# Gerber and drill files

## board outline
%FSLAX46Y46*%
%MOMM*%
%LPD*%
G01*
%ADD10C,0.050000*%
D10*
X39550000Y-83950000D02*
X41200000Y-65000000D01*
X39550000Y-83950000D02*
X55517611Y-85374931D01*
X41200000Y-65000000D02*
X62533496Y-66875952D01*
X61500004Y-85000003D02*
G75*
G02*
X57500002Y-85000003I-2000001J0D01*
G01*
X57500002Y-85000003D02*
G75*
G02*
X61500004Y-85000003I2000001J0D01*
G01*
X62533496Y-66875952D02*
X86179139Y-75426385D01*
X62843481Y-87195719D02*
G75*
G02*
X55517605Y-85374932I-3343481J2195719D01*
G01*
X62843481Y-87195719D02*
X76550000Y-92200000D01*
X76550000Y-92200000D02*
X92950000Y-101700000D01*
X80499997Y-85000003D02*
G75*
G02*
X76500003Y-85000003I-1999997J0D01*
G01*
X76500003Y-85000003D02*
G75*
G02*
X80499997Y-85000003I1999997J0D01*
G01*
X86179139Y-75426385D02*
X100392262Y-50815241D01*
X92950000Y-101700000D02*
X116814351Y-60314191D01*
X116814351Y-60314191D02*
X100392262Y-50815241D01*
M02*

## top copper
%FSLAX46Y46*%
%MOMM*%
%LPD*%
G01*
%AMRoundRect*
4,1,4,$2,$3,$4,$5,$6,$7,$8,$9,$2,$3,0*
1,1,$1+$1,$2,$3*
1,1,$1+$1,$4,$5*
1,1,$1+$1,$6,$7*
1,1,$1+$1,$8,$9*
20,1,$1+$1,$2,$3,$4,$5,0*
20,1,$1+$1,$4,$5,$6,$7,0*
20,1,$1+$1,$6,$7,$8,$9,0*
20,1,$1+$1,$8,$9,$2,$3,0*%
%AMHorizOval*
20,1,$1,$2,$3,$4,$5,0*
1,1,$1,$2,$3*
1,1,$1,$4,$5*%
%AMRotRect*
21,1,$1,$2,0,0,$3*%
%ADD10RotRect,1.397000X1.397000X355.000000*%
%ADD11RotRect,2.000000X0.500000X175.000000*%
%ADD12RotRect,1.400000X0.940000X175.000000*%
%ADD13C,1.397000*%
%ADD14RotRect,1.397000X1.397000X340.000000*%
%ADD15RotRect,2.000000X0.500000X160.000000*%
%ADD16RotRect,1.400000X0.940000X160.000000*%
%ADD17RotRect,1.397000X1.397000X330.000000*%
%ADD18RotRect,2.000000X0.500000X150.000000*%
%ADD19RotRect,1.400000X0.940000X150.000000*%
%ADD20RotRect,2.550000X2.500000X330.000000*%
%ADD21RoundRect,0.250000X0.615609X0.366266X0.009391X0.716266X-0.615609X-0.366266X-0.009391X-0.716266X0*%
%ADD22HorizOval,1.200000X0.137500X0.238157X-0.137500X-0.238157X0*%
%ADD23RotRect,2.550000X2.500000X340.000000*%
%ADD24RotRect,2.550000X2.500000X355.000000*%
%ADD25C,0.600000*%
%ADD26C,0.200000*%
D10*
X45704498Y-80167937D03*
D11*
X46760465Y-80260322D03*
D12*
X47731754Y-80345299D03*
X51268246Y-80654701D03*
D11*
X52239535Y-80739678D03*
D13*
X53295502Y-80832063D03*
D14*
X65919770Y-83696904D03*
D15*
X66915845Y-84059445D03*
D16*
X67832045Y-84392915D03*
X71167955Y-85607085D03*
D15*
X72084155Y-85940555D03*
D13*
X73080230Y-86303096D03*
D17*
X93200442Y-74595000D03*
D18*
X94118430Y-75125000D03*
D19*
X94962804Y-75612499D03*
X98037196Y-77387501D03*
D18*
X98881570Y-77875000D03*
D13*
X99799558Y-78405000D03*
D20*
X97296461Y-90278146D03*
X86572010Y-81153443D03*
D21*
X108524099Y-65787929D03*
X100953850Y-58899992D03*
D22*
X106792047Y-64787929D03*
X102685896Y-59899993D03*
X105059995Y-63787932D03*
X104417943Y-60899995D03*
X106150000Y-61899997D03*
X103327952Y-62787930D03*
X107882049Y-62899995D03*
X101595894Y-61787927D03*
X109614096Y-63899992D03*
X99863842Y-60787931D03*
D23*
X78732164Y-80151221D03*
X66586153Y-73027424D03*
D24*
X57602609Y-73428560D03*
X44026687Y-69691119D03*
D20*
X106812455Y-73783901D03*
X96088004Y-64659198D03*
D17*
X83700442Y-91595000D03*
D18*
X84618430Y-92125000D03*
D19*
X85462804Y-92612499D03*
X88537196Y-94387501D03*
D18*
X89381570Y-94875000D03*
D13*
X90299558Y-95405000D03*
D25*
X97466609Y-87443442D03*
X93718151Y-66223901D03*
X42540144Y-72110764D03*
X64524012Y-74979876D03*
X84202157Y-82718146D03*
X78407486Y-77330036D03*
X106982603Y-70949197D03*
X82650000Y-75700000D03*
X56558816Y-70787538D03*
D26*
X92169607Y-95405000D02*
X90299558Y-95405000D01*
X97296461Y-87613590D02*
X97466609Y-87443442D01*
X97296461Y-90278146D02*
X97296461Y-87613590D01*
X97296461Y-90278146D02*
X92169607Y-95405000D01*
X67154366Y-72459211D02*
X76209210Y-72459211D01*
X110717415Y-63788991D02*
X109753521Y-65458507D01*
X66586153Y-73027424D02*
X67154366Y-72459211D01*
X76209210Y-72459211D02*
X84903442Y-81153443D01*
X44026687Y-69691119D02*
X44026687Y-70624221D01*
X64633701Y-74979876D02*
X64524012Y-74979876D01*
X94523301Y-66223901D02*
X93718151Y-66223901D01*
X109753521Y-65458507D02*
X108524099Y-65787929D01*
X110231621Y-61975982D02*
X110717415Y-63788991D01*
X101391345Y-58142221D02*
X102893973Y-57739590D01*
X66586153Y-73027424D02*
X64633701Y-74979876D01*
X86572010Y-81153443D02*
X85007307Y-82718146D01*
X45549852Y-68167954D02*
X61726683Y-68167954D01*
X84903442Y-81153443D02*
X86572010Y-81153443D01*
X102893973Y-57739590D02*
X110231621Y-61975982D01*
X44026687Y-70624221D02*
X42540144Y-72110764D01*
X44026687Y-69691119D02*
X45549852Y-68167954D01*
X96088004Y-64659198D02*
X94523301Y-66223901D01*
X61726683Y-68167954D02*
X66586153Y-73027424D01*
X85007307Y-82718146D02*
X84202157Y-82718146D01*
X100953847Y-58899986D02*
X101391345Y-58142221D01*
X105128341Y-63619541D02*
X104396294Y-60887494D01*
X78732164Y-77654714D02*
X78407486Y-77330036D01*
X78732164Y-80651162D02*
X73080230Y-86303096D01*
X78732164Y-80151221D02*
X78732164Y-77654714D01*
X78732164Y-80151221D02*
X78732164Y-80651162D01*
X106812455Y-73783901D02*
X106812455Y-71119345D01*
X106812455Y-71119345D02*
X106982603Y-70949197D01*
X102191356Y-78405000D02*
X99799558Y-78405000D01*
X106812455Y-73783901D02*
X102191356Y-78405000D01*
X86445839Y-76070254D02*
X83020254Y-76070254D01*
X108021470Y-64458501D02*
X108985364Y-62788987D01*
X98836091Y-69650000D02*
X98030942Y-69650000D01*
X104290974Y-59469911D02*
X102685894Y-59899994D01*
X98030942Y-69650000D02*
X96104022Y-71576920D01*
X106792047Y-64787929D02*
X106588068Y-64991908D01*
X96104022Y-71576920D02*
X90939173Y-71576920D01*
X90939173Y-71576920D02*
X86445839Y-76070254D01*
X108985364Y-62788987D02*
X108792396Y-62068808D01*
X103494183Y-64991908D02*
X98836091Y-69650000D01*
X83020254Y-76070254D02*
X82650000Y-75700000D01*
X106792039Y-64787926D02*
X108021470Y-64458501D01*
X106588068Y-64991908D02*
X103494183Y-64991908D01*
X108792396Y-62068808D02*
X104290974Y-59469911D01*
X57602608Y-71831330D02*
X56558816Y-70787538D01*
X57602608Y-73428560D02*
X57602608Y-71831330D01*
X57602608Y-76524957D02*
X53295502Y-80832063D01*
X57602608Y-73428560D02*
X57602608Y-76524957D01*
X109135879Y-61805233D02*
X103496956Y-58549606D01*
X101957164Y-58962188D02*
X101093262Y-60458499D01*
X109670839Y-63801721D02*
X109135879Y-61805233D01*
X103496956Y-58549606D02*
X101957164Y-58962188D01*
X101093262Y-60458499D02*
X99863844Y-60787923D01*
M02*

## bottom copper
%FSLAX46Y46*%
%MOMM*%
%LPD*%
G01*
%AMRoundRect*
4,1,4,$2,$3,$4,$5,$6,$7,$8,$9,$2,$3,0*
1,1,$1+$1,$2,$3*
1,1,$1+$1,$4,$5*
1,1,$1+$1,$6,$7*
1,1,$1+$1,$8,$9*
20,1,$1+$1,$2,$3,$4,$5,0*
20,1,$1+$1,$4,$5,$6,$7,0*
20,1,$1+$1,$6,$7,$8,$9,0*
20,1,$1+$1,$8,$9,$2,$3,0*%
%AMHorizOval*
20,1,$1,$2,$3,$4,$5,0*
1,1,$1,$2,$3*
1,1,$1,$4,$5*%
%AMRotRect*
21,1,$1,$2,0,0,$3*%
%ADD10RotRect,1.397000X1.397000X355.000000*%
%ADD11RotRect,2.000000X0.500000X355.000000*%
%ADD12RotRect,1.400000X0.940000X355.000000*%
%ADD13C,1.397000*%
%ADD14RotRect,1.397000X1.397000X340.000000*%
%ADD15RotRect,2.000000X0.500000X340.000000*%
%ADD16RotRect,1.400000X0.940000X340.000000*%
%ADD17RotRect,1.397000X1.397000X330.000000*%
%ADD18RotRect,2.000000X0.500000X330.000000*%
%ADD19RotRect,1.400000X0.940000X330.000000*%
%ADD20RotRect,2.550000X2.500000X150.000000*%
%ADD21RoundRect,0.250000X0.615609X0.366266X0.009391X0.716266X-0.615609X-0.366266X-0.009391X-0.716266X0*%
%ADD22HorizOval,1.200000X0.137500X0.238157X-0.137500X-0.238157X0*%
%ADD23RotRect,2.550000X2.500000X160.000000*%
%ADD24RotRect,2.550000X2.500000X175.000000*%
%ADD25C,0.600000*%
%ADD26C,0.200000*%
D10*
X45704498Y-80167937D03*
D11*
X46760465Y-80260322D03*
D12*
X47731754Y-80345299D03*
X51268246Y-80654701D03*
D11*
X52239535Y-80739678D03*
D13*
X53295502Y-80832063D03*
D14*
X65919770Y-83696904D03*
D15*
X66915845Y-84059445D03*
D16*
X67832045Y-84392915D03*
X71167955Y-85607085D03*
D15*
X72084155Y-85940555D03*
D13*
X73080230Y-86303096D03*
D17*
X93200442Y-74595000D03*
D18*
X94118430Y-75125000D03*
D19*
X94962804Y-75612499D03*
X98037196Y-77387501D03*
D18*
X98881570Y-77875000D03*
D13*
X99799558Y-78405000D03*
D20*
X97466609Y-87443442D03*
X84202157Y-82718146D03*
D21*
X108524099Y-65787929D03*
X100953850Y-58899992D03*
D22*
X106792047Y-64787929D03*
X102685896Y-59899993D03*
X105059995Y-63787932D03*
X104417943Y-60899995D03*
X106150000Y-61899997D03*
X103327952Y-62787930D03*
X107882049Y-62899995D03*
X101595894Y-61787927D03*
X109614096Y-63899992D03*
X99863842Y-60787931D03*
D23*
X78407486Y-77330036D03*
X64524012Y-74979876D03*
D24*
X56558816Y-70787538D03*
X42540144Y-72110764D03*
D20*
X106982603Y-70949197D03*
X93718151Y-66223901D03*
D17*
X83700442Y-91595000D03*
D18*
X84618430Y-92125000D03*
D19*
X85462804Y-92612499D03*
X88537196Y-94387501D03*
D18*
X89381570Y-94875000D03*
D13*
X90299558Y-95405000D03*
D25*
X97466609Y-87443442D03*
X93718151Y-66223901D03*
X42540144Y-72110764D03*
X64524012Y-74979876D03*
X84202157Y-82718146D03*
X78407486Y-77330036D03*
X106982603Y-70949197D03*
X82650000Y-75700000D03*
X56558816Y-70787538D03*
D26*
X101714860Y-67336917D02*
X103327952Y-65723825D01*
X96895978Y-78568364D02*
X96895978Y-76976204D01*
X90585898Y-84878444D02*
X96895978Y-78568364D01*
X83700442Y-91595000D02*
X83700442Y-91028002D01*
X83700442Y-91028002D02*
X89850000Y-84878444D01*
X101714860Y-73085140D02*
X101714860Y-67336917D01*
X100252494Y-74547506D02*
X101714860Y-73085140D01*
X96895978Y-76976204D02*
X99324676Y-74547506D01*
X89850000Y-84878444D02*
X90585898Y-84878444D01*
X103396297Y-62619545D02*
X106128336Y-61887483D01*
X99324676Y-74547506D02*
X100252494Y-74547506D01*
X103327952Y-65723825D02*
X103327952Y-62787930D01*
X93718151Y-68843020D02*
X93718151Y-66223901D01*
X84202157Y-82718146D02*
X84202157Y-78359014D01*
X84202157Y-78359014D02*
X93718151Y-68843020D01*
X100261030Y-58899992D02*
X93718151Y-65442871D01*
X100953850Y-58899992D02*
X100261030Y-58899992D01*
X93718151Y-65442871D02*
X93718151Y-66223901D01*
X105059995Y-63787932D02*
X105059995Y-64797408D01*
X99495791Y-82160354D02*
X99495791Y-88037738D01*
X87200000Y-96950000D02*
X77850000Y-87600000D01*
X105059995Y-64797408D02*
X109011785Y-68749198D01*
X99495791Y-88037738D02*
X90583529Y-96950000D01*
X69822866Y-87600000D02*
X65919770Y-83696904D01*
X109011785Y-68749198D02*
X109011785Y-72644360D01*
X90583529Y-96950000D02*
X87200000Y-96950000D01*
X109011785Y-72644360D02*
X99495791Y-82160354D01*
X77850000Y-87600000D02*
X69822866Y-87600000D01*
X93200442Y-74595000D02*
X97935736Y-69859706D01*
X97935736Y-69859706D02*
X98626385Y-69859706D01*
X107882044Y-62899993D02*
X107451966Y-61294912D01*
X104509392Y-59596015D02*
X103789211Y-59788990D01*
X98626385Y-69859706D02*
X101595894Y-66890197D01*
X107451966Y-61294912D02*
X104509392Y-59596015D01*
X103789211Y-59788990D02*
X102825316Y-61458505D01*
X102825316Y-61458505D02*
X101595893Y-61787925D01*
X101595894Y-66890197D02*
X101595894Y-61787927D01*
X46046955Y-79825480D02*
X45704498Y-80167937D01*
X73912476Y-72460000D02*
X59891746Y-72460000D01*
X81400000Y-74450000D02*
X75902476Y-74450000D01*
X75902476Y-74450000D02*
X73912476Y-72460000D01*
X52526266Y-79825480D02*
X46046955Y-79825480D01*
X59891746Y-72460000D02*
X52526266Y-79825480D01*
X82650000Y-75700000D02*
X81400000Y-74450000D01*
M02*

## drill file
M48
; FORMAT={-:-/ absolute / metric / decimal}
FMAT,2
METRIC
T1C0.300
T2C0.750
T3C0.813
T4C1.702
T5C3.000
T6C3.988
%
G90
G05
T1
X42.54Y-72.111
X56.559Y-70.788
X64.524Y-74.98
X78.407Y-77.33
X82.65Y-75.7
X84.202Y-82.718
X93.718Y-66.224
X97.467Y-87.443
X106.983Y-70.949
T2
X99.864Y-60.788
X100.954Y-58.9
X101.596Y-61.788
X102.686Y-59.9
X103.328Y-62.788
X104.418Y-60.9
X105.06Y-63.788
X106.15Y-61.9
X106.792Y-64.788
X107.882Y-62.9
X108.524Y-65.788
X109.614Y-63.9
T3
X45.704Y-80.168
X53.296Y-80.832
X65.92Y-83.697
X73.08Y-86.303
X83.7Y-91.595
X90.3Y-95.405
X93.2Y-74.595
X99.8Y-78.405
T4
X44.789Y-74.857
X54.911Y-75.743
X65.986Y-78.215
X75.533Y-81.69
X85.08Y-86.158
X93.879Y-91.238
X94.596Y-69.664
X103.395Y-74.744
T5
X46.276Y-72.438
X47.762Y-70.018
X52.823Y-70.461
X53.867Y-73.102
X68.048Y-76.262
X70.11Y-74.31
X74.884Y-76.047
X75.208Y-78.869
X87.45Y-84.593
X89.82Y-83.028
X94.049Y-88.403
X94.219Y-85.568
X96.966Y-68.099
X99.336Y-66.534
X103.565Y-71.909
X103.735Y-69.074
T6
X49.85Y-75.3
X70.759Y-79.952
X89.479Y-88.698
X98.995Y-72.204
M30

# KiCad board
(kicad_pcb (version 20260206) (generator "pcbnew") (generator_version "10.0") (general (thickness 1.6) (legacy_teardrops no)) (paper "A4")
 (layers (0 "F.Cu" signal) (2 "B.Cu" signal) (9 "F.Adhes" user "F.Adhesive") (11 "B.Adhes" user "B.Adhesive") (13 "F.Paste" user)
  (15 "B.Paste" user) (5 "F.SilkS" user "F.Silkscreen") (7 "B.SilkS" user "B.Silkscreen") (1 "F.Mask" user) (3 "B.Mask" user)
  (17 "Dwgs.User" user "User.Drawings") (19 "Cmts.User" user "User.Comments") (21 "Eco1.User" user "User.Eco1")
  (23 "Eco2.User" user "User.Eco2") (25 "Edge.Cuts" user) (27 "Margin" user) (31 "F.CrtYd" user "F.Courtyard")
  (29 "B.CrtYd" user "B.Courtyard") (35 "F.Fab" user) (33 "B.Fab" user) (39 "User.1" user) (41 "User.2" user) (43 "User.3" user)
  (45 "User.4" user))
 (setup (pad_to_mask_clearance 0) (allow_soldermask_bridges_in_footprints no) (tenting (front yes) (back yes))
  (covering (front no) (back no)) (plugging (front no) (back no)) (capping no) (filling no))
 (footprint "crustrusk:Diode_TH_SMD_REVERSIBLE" (layer "F.Cu") (at 49.5 80.5 -5)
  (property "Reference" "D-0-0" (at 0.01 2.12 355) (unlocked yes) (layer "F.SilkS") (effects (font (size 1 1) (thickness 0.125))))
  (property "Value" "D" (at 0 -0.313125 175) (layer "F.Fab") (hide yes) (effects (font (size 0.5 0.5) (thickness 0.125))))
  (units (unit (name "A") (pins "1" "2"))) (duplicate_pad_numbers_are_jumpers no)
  (pad "1" thru_hole rect (at -3.81 0 355) (size 1.397 1.397) (drill 0.8128) (layers "*.Cu" "*.Mask") (remove_unused_layers no)
   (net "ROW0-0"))
  (pad "1" smd rect (at -2.75 0 175) (size 2 0.5) (layers "F.Cu") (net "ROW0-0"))
  (pad "1" smd rect (at -2.75 0 355) (size 2 0.5) (layers "B.Cu") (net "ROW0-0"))
  (pad "1" smd rect (at -1.775 0 175) (size 1.4 0.94) (layers "F.Cu" "F.Mask" "F.Paste") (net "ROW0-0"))
  (pad "1" smd rect (at -1.775 0 355) (size 1.4 0.94) (layers "B.Cu" "B.Mask" "B.Paste") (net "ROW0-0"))
  (pad "2" smd rect (at 1.775 0 175) (size 1.4 0.94) (layers "F.Cu" "F.Mask" "F.Paste") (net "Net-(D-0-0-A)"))
  (pad "2" smd rect (at 1.775 0 355) (size 1.4 0.94) (layers "B.Cu" "B.Mask" "B.Paste") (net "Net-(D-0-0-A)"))
  (pad "2" smd rect (at 2.75 0 175) (size 2 0.5) (layers "F.Cu") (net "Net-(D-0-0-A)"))
  (pad "2" smd rect (at 2.75 0 355) (size 2 0.5) (layers "B.Cu") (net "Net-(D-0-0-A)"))
  (pad "2" thru_hole circle (at 3.81 0 355) (size 1.397 1.397) (drill 0.8128) (layers "*.Cu" "*.Mask") (remove_unused_layers no)
   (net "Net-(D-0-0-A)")))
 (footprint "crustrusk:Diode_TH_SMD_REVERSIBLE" (layer "F.Cu") (at 69.5 85 -20)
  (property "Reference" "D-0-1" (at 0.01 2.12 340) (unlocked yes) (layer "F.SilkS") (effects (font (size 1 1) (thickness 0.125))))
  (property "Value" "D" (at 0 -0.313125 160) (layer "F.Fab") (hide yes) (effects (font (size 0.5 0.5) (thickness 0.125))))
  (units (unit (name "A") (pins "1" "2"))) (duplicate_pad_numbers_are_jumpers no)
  (pad "1" thru_hole rect (at -3.810001 0.000001 340) (size 1.397 1.397) (drill 0.8128) (layers "*.Cu" "*.Mask") (remove_unused_layers no)
   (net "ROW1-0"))
  (pad "1" smd rect (at -2.75 0 160) (size 2 0.5) (layers "F.Cu") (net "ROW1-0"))
  (pad "1" smd rect (at -2.75 0 340) (size 2 0.5) (layers "B.Cu") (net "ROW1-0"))
  (pad "1" smd rect (at -1.775 0.000001 160) (size 1.4 0.94) (layers "F.Cu" "F.Mask" "F.Paste") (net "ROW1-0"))
  (pad "1" smd rect (at -1.775 0.000001 340) (size 1.4 0.94) (layers "B.Cu" "B.Mask" "B.Paste") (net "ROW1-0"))
  (pad "2" smd rect (at 1.775 -0.000001 160) (size 1.4 0.94) (layers "F.Cu" "F.Mask" "F.Paste") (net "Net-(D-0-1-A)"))
  (pad "2" smd rect (at 1.775 -0.000001 340) (size 1.4 0.94) (layers "B.Cu" "B.Mask" "B.Paste") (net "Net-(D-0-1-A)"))
  (pad "2" smd rect (at 2.75 0 160) (size 2 0.5) (layers "F.Cu") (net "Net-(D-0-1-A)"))
  (pad "2" smd rect (at 2.75 0 340) (size 2 0.5) (layers "B.Cu") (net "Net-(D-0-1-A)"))
  (pad "2" thru_hole circle (at 3.810001 -0.000001 340) (size 1.397 1.397) (drill 0.8128) (layers "*.Cu" "*.Mask") (remove_unused_layers no)
   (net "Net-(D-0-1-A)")))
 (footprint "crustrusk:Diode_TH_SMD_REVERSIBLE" (layer "F.Cu") (at 96.5 76.5 -30)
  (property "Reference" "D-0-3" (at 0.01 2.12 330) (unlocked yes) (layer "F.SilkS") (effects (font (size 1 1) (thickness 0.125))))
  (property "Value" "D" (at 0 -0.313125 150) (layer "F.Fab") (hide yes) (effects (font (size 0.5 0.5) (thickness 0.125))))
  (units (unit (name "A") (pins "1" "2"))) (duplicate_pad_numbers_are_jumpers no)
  (pad "1" thru_hole rect (at -3.810001 0.000001 330) (size 1.397 1.397) (drill 0.8128) (layers "*.Cu" "*.Mask") (remove_unused_layers no)
   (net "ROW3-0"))
  (pad "1" smd rect (at -2.75 0 150) (size 2 0.5) (layers "F.Cu") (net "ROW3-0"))
  (pad "1" smd rect (at -2.75 0 330) (size 2 0.5) (layers "B.Cu") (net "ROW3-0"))
  (pad "1" smd rect (at -1.775001 0 150) (size 1.4 0.94) (layers "F.Cu" "F.Mask" "F.Paste") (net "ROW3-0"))
  (pad "1" smd rect (at -1.775001 0 330) (size 1.4 0.94) (layers "B.Cu" "B.Mask" "B.Paste") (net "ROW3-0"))
  (pad "2" smd rect (at 1.775001 0 150) (size 1.4 0.94) (layers "F.Cu" "F.Mask" "F.Paste") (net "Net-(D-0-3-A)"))
  (pad "2" smd rect (at 1.775001 0 330) (size 1.4 0.94) (layers "B.Cu" "B.Mask" "B.Paste") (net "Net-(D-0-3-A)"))
  (pad "2" smd rect (at 2.75 0 150) (size 2 0.5) (layers "F.Cu") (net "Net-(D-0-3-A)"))
  (pad "2" smd rect (at 2.75 0 330) (size 2 0.5) (layers "B.Cu") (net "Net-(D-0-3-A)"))
  (pad "2" thru_hole circle (at 3.810001 -0.000001 330) (size 1.397 1.397) (drill 0.8128) (layers "*.Cu" "*.Mask") (remove_unused_layers no)
   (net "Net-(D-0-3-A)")))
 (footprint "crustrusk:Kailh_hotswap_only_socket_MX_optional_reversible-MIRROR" (layer "F.Cu") (at 89.479309 88.697851 -30)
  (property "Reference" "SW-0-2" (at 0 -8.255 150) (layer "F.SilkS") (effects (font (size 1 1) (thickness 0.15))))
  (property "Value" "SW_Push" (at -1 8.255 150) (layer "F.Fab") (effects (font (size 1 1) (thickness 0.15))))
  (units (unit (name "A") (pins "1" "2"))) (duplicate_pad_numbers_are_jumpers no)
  (pad "" np_thru_hole circle (at -5.08 0 330) (size 1.7018 1.7018) (drill 1.7018) (layers "*.Cu" "*.Mask"))
  (pad "" np_thru_hole circle (at -3.81 -2.54 150) (size 3 3) (drill 3) (layers "*.Cu" "*.Mask"))
  (pad "" np_thru_hole circle (at -2.54 -5.079997 330) (size 3 3) (drill 3) (layers "*.Cu" "*.Mask"))
  (pad "" np_thru_hole circle (at 0 0 330) (size 3.9878 3.9878) (drill 3.9878) (layers "*.Cu" "*.Mask"))
  (pad "" np_thru_hole circle (at 2.540002 -5.080001 150) (size 3 3) (drill 3) (layers "*.Cu" "*.Mask"))
  (pad "" np_thru_hole circle (at 3.81 -2.540001 330) (size 3 3) (drill 3) (layers "*.Cu" "*.Mask"))
  (pad "" np_thru_hole circle (at 5.08 0 330) (size 1.7018 1.7018) (drill 1.7018) (layers "*.Cu" "*.Mask"))
  (pad "1" smd rect (at 6.29 -5.08 150) (size 2.55 2.5) (layers "B.Cu" "B.Mask" "B.Paste") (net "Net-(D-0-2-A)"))
  (pad "1" smd rect (at 7.56 -2.54 330) (size 2.55 2.5) (layers "F.Cu" "F.Mask" "F.Paste") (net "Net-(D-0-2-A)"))
  (pad "2" smd rect (at -7.56 -2.54 150) (size 2.55 2.5) (layers "B.Cu" "B.Mask" "B.Paste") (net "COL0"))
  (pad "2" smd rect (at -6.289999 -5.079999 330) (size 2.55 2.5) (layers "F.Cu" "F.Mask" "F.Paste") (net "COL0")))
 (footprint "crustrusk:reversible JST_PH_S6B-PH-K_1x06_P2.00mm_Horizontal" (layer "F.Cu") (at 108.524099 65.787929 150)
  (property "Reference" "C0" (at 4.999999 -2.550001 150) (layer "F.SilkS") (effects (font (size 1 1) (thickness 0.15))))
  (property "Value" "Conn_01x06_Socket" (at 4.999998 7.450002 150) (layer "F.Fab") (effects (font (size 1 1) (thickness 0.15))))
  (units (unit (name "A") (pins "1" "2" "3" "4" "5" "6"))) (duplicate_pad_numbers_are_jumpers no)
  (pad "1" thru_hole roundrect (at 0 0 150) (size 1.2 1.75) (drill 0.75) (layers "*.Cu" "*.Mask") (remove_unused_layers no)
   (roundrect_rratio 0.208333) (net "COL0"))
  (pad "1" thru_hole roundrect (at 9.999996 2.180004 150) (size 1.2 1.75) (drill 0.75) (layers "*.Cu" "*.Mask") (remove_unused_layers no)
   (roundrect_rratio 0.208333) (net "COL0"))
  (pad "2" thru_hole oval (at 2.000001 -0.000001 150) (size 1.2 1.75) (drill 0.75) (layers "*.Cu" "*.Mask") (remove_unused_layers no)
   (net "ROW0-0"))
  (pad "2" thru_hole oval (at 8 2.180001 150) (size 1.2 1.75) (drill 0.75) (layers "*.Cu" "*.Mask") (remove_unused_layers no) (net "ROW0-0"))
  (pad "3" thru_hole oval (at 4.000001 -0.000004 150) (size 1.2 1.75) (drill 0.75) (layers "*.Cu" "*.Mask") (remove_unused_layers no)
   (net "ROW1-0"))
  (pad "3" thru_hole oval (at 6.000002 2.179997 150) (size 1.2 1.75) (drill 0.75) (layers "*.Cu" "*.Mask") (remove_unused_layers no)
   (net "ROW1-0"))
  (pad "4" thru_hole oval (at 3.999996 2.179998 150) (size 1.2 1.75) (drill 0.75) (layers "*.Cu" "*.Mask") (remove_unused_layers no)
   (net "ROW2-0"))
  (pad "4" thru_hole oval (at 5.999995 0.000002 150) (size 1.2 1.75) (drill 0.75) (layers "*.Cu" "*.Mask") (remove_unused_layers no)
   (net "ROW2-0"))
  (pad "5" thru_hole oval (at 1.999999 2.179999 150) (size 1.2 1.75) (drill 0.75) (layers "*.Cu" "*.Mask") (remove_unused_layers no)
   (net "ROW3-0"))
  (pad "5" thru_hole oval (at 8.000003 0.000001 150) (size 1.2 1.75) (drill 0.75) (layers "*.Cu" "*.Mask") (remove_unused_layers no)
   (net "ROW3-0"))
  (pad "6" thru_hole oval (at 0.000003 2.18 150) (size 1.2 1.75) (drill 0.75) (layers "*.Cu" "*.Mask") (remove_unused_layers no)
   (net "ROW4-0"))
  (pad "6" thru_hole oval (at 10.000002 -0.000003 150) (size 1.2 1.75) (drill 0.75) (layers "*.Cu" "*.Mask") (remove_unused_layers no)
   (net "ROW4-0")))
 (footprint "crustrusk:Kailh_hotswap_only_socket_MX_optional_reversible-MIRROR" (layer "F.Cu") (at 70.759357 79.952368 -20)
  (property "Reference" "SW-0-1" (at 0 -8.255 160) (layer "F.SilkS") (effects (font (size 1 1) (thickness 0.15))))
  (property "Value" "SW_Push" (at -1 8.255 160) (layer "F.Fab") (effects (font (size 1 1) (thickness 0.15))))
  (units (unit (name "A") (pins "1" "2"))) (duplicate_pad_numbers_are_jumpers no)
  (pad "" np_thru_hole circle (at -5.08 0 340) (size 1.7018 1.7018) (drill 1.7018) (layers "*.Cu" "*.Mask"))
  (pad "" np_thru_hole circle (at -3.81 -2.54 160) (size 3 3) (drill 3) (layers "*.Cu" "*.Mask"))
  (pad "" np_thru_hole circle (at -2.54 -5.079998 340) (size 3 3) (drill 3) (layers "*.Cu" "*.Mask"))
  (pad "" np_thru_hole circle (at 0 0 340) (size 3.9878 3.9878) (drill 3.9878) (layers "*.Cu" "*.Mask"))
  (pad "" np_thru_hole circle (at 2.540002 -5.080001 160) (size 3 3) (drill 3) (layers "*.Cu" "*.Mask"))
  (pad "" np_thru_hole circle (at 3.81 -2.54 340) (size 3 3) (drill 3) (layers "*.Cu" "*.Mask"))
  (pad "" np_thru_hole circle (at 5.08 0 340) (size 1.7018 1.7018) (drill 1.7018) (layers "*.Cu" "*.Mask"))
  (pad "1" smd rect (at 6.29 -5.08 160) (size 2.55 2.5) (layers "B.Cu" "B.Mask" "B.Paste") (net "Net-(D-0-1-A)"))
  (pad "1" smd rect (at 7.56 -2.54 340) (size 2.55 2.5) (layers "F.Cu" "F.Mask" "F.Paste") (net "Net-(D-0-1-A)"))
  (pad "2" smd rect (at -7.56 -2.54 160) (size 2.55 2.5) (layers "B.Cu" "B.Mask" "B.Paste") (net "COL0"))
  (pad "2" smd rect (at -6.289999 -5.079999 340) (size 2.55 2.5) (layers "F.Cu" "F.Mask" "F.Paste") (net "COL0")))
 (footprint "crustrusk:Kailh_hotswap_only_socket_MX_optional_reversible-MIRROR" (layer "F.Cu") (at 49.85 75.299997 -5)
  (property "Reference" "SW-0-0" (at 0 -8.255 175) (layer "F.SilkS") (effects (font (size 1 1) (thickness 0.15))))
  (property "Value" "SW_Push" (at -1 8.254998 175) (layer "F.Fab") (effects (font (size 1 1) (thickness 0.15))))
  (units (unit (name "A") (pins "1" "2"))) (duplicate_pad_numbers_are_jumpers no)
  (pad "" np_thru_hole circle (at -5.08 0 355) (size 1.7018 1.7018) (drill 1.7018) (layers "*.Cu" "*.Mask"))
  (pad "" np_thru_hole circle (at -3.81 -2.54 175) (size 3 3) (drill 3) (layers "*.Cu" "*.Mask"))
  (pad "" np_thru_hole circle (at -2.54 -5.079998 355) (size 3 3) (drill 3) (layers "*.Cu" "*.Mask"))
  (pad "" np_thru_hole circle (at 0 0 355) (size 3.9878 3.9878) (drill 3.9878) (layers "*.Cu" "*.Mask"))
  (pad "" np_thru_hole circle (at 2.540002 -5.080001 175) (size 3 3) (drill 3) (layers "*.Cu" "*.Mask"))
  (pad "" np_thru_hole circle (at 3.81 -2.54 355) (size 3 3) (drill 3) (layers "*.Cu" "*.Mask"))
  (pad "" np_thru_hole circle (at 5.08 0 355) (size 1.7018 1.7018) (drill 1.7018) (layers "*.Cu" "*.Mask"))
  (pad "1" smd rect (at 6.29 -5.08 175) (size 2.55 2.5) (layers "B.Cu" "B.Mask" "B.Paste") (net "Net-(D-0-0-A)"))
  (pad "1" smd rect (at 7.560001 -2.54 355) (size 2.55 2.5) (layers "F.Cu" "F.Mask" "F.Paste") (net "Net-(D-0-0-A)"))
  (pad "2" smd rect (at -7.56 -2.540001 175) (size 2.55 2.5) (layers "B.Cu" "B.Mask" "B.Paste") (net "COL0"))
  (pad "2" smd rect (at -6.289999 -5.079999 355) (size 2.55 2.5) (layers "F.Cu" "F.Mask" "F.Paste") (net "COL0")))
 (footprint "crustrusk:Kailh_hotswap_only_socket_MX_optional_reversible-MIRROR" (layer "F.Cu") (at 98.995303 72.203606 -30)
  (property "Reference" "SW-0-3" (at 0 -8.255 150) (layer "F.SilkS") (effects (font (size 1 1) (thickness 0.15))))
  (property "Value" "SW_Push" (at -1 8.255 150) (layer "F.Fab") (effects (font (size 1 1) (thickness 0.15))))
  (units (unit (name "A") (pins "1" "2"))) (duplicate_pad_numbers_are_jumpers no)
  (pad "" np_thru_hole circle (at -5.08 0 330) (size 1.7018 1.7018) (drill 1.7018) (layers "*.Cu" "*.Mask"))
  (pad "" np_thru_hole circle (at -3.81 -2.54 150) (size 3 3) (drill 3) (layers "*.Cu" "*.Mask"))
  (pad "" np_thru_hole circle (at -2.54 -5.079997 330) (size 3 3) (drill 3) (layers "*.Cu" "*.Mask"))
  (pad "" np_thru_hole circle (at 0 0 330) (size 3.9878 3.9878) (drill 3.9878) (layers "*.Cu" "*.Mask"))
  (pad "" np_thru_hole circle (at 2.540002 -5.080001 150) (size 3 3) (drill 3) (layers "*.Cu" "*.Mask"))
  (pad "" np_thru_hole circle (at 3.81 -2.540001 330) (size 3 3) (drill 3) (layers "*.Cu" "*.Mask"))
  (pad "" np_thru_hole circle (at 5.08 0 330) (size 1.7018 1.7018) (drill 1.7018) (layers "*.Cu" "*.Mask"))
  (pad "1" smd rect (at 6.29 -5.08 150) (size 2.55 2.5) (layers "B.Cu" "B.Mask" "B.Paste") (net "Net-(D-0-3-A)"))
  (pad "1" smd rect (at 7.56 -2.54 330) (size 2.55 2.5) (layers "F.Cu" "F.Mask" "F.Paste") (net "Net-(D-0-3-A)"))
  (pad "2" smd rect (at -7.56 -2.54 150) (size 2.55 2.5) (layers "B.Cu" "B.Mask" "B.Paste") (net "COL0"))
  (pad "2" smd rect (at -6.289999 -5.079999 330) (size 2.55 2.5) (layers "F.Cu" "F.Mask" "F.Paste") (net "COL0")))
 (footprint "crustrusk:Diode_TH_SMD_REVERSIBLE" (layer "F.Cu") (at 87 93.5 -30)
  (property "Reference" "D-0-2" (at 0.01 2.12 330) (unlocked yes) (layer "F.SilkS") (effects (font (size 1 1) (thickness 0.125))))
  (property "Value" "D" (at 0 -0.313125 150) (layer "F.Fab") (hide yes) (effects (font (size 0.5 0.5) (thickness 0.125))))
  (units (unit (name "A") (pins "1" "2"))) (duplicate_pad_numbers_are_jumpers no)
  (pad "1" thru_hole rect (at -3.810001 0.000001 330) (size 1.397 1.397) (drill 0.8128) (layers "*.Cu" "*.Mask") (remove_unused_layers no)
   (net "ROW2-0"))
  (pad "1" smd rect (at -2.75 0 150) (size 2 0.5) (layers "F.Cu") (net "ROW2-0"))
  (pad "1" smd rect (at -2.75 0 330) (size 2 0.5) (layers "B.Cu") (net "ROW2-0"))
  (pad "1" smd rect (at -1.775001 0 150) (size 1.4 0.94) (layers "F.Cu" "F.Mask" "F.Paste") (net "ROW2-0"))
  (pad "1" smd rect (at -1.775001 0 330) (size 1.4 0.94) (layers "B.Cu" "B.Mask" "B.Paste") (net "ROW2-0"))
  (pad "2" smd rect (at 1.775001 0 150) (size 1.4 0.94) (layers "F.Cu" "F.Mask" "F.Paste") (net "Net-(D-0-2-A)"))
  (pad "2" smd rect (at 1.775001 0 330) (size 1.4 0.94) (layers "B.Cu" "B.Mask" "B.Paste") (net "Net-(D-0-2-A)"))
  (pad "2" smd rect (at 2.75 0 150) (size 2 0.5) (layers "F.Cu") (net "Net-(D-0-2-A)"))
  (pad "2" smd rect (at 2.75 0 330) (size 2 0.5) (layers "B.Cu") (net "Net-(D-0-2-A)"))
  (pad "2" thru_hole circle (at 3.810001 -0.000001 330) (size 1.397 1.397) (drill 0.8128) (layers "*.Cu" "*.Mask") (remove_unused_layers no)
   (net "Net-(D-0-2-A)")))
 (gr_line (start 39.55 83.95) (end 41.2 65) (stroke (width 0.05) (type default)) (layer "Edge.Cuts"))
 (gr_line (start 39.55 83.95) (end 55.517611 85.374931) (stroke (width 0.05) (type default)) (layer "Edge.Cuts"))
 (gr_line (start 41.2 65) (end 62.533496 66.875952) (stroke (width 0.05) (type default)) (layer "Edge.Cuts"))
 (gr_circle (center 59.500003 85.000003) (end 57.500002 85.000003) (stroke (width 0.05) (type default)) (fill no) (layer "Edge.Cuts"))
 (gr_line (start 62.533496 66.875952) (end 86.179139 75.426385) (stroke (width 0.05) (type default)) (layer "Edge.Cuts"))
 (gr_arc (start 62.843481 87.195719) (mid 58.535187 88.881903) (end 55.517611 85.374931) (stroke (width 0.05) (type default))
  (layer "Edge.Cuts"))
 (gr_line (start 62.843481 87.195719) (end 76.55 92.2) (stroke (width 0.05) (type default)) (layer "Edge.Cuts"))
 (gr_line (start 76.55 92.2) (end 92.95 101.7) (stroke (width 0.05) (type default)) (layer "Edge.Cuts"))
 (gr_circle (center 78.5 85.000003) (end 76.500003 85.000003) (stroke (width 0.05) (type default)) (fill no) (layer "Edge.Cuts"))
 (gr_line (start 86.179139 75.426385) (end 100.392262 50.815241) (stroke (width 0.05) (type default)) (layer "Edge.Cuts"))
 (gr_line (start 92.95 101.7) (end 116.814351 60.314191) (stroke (width 0.05) (type default)) (layer "Edge.Cuts"))
 (gr_line (start 116.814351 60.314191) (end 100.392262 50.815241) (stroke (width 0.05) (type default)) (layer "Edge.Cuts"))
 (segment (start 101.71486 67.336917) (end 103.327952 65.723825) (width 0.2) (layer "B.Cu") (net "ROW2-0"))
 (segment (start 96.895978 78.568364) (end 96.895978 76.976204) (width 0.2) (layer "B.Cu") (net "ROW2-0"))
 (segment (start 90.585898 84.878444) (end 96.895978 78.568364) (width 0.2) (layer "B.Cu") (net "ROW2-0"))
 (segment (start 83.700442 91.595) (end 83.700442 91.028002) (width 0.2) (layer "B.Cu") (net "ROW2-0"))
 (segment (start 83.700442 91.028002) (end 89.85 84.878444) (width 0.2) (layer "B.Cu") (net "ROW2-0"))
 (segment (start 101.71486 73.08514) (end 101.71486 67.336917) (width 0.2) (layer "B.Cu") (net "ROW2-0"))
 (segment (start 100.252494 74.547506) (end 101.71486 73.08514) (width 0.2) (layer "B.Cu") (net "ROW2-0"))
 (segment (start 96.895978 76.976204) (end 99.324676 74.547506) (width 0.2) (layer "B.Cu") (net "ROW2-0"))
 (segment (start 89.85 84.878444) (end 90.585898 84.878444) (width 0.2) (layer "B.Cu") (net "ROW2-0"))
 (segment (start 103.396297 62.619545) (end 106.128336 61.887483) (width 0.2) (layer "B.Cu") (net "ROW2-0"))
 (segment (start 99.324676 74.547506) (end 100.252494 74.547506) (width 0.2) (layer "B.Cu") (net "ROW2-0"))
 (segment (start 103.327952 65.723825) (end 103.327952 62.78793) (width 0.2) (layer "B.Cu") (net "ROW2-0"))
 (segment (start 92.169607 95.405) (end 90.299558 95.405) (width 0.2) (layer "F.Cu") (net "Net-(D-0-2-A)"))
 (segment (start 97.296461 87.61359) (end 97.466609 87.443442) (width 0.2) (layer "F.Cu") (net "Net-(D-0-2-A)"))
 (segment (start 97.296461 90.278146) (end 97.296461 87.61359) (width 0.2) (layer "F.Cu") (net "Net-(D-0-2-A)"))
 (segment (start 97.296461 90.278146) (end 92.169607 95.405) (width 0.2) (layer "F.Cu") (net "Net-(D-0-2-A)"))
 (via (at 97.466609 87.443442) (size 0.6) (drill 0.3) (layers "F.Cu" "B.Cu") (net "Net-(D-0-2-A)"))
 (segment (start 67.154366 72.459211) (end 76.20921 72.459211) (width 0.2) (layer "F.Cu") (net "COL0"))
 (segment (start 110.717415 63.788991) (end 109.753521 65.458507) (width 0.2) (layer "F.Cu") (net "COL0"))
 (segment (start 66.586153 73.027424) (end 67.154366 72.459211) (width 0.2) (layer "F.Cu") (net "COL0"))
 (segment (start 76.20921 72.459211) (end 84.903442 81.153443) (width 0.2) (layer "F.Cu") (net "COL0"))
 (segment (start 44.026687 69.691119) (end 44.026687 70.624221) (width 0.2) (layer "F.Cu") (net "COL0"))
 (segment (start 64.633701 74.979876) (end 64.524012 74.979876) (width 0.2) (layer "F.Cu") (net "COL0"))
 (segment (start 94.523301 66.223901) (end 93.718151 66.223901) (width 0.2) (layer "F.Cu") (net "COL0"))
 (segment (start 109.753521 65.458507) (end 108.524099 65.787929) (width 0.2) (layer "F.Cu") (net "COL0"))
 (segment (start 110.231621 61.975982) (end 110.717415 63.788991) (width 0.2) (layer "F.Cu") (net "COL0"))
 (segment (start 101.391345 58.142221) (end 102.893973 57.73959) (width 0.2) (layer "F.Cu") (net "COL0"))
 (segment (start 66.586153 73.027424) (end 64.633701 74.979876) (width 0.2) (layer "F.Cu") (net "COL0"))
 (segment (start 86.57201 81.153443) (end 85.007307 82.718146) (width 0.2) (layer "F.Cu") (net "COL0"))
 (segment (start 45.549852 68.167954) (end 61.726683 68.167954) (width 0.2) (layer "F.Cu") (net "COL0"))
 (segment (start 84.903442 81.153443) (end 86.57201 81.153443) (width 0.2) (layer "F.Cu") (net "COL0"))
 (segment (start 102.893973 57.73959) (end 110.231621 61.975982) (width 0.2) (layer "F.Cu") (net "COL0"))
 (segment (start 44.026687 70.624221) (end 42.540144 72.110764) (width 0.2) (layer "F.Cu") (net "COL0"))
 (segment (start 44.026687 69.691119) (end 45.549852 68.167954) (width 0.2) (layer "F.Cu") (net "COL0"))
 (segment (start 96.088004 64.659198) (end 94.523301 66.223901) (width 0.2) (layer "F.Cu") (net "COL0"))
 (segment (start 61.726683 68.167954) (end 66.586153 73.027424) (width 0.2) (layer "F.Cu") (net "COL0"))
 (segment (start 85.007307 82.718146) (end 84.202157 82.718146) (width 0.2) (layer "F.Cu") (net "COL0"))
 (segment (start 100.953847 58.899986) (end 101.391345 58.142221) (width 0.2) (layer "F.Cu") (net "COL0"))
 (via (at 93.718151 66.223901) (size 0.6) (drill 0.3) (layers "F.Cu" "B.Cu") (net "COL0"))
 (via (at 42.540144 72.110764) (size 0.6) (drill 0.3) (layers "F.Cu" "B.Cu") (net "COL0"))
 (via (at 64.524012 74.979876) (size 0.6) (drill 0.3) (layers "F.Cu" "B.Cu") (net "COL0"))
 (via (at 84.202157 82.718146) (size 0.6) (drill 0.3) (layers "F.Cu" "B.Cu") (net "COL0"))
 (segment (start 93.718151 68.84302) (end 93.718151 66.223901) (width 0.2) (layer "B.Cu") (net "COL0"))
 (segment (start 84.202157 82.718146) (end 84.202157 78.359014) (width 0.2) (layer "B.Cu") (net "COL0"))
 (segment (start 84.202157 78.359014) (end 93.718151 68.84302) (width 0.2) (layer "B.Cu") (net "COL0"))
 (segment (start 100.26103 58.899992) (end 93.718151 65.442871) (width 0.2) (layer "B.Cu") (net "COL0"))
 (segment (start 100.95385 58.899992) (end 100.26103 58.899992) (width 0.2) (layer "B.Cu") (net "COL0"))
 (segment (start 93.718151 65.442871) (end 93.718151 66.223901) (width 0.2) (layer "B.Cu") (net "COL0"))
 (segment (start 105.128341 63.619541) (end 104.396294 60.887494) (width 0.2) (layer "F.Cu") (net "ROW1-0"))
 (segment (start 105.059995 63.787932) (end 105.059995 64.797408) (width 0.2) (layer "B.Cu") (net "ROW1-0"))
 (segment (start 99.495791 82.160354) (end 99.495791 88.037738) (width 0.2) (layer "B.Cu") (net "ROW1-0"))
 (segment (start 87.2 96.95) (end 77.85 87.6) (width 0.2) (layer "B.Cu") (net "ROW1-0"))
 (segment (start 105.059995 64.797408) (end 109.011785 68.749198) (width 0.2) (layer "B.Cu") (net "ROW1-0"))
 (segment (start 99.495791 88.037738) (end 90.583529 96.95) (width 0.2) (layer "B.Cu") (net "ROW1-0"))
 (segment (start 69.822866 87.6) (end 65.91977 83.696904) (width 0.2) (layer "B.Cu") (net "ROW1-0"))
 (segment (start 109.011785 68.749198) (end 109.011785 72.64436) (width 0.2) (layer "B.Cu") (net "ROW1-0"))
 (segment (start 90.583529 96.95) (end 87.2 96.95) (width 0.2) (layer "B.Cu") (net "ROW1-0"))
 (segment (start 109.011785 72.64436) (end 99.495791 82.160354) (width 0.2) (layer "B.Cu") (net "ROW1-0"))
 (segment (start 77.85 87.6) (end 69.822866 87.6) (width 0.2) (layer "B.Cu") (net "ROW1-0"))
 (segment (start 78.732164 77.654714) (end 78.407486 77.330036) (width 0.2) (layer "F.Cu") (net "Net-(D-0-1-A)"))
 (segment (start 78.732164 80.651162) (end 73.08023 86.303096) (width 0.2) (layer "F.Cu") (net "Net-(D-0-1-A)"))
 (segment (start 78.732164 80.151221) (end 78.732164 77.654714) (width 0.2) (layer "F.Cu") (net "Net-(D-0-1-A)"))
 (segment (start 78.732164 80.151221) (end 78.732164 80.651162) (width 0.2) (layer "F.Cu") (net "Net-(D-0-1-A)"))
 (via (at 78.407486 77.330036) (size 0.6) (drill 0.3) (layers "F.Cu" "B.Cu") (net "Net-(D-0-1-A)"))
 (segment (start 93.200442 74.595) (end 97.935736 69.859706) (width 0.2) (layer "B.Cu") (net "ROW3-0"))
 (segment (start 97.935736 69.859706) (end 98.626385 69.859706) (width 0.2) (layer "B.Cu") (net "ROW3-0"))
 (segment (start 107.882044 62.899993) (end 107.451966 61.294912) (width 0.2) (layer "B.Cu") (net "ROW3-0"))
 (segment (start 104.509392 59.596015) (end 103.789211 59.78899) (width 0.2) (layer "B.Cu") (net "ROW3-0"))
 (segment (start 98.626385 69.859706) (end 101.595894 66.890197) (width 0.2) (layer "B.Cu") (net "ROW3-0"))
 (segment (start 107.451966 61.294912) (end 104.509392 59.596015) (width 0.2) (layer "B.Cu") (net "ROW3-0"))
 (segment (start 103.789211 59.78899) (end 102.825316 61.458505) (width 0.2) (layer "B.Cu") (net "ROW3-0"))
 (segment (start 102.825316 61.458505) (end 101.595893 61.787925) (width 0.2) (layer "B.Cu") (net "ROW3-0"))
 (segment (start 101.595894 66.890197) (end 101.595894 61.787927) (width 0.2) (layer "B.Cu") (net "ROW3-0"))
 (segment (start 106.812455 73.783901) (end 106.812455 71.119345) (width 0.2) (layer "F.Cu") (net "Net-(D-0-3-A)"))
 (segment (start 106.812455 71.119345) (end 106.982603 70.949197) (width 0.2) (layer "F.Cu") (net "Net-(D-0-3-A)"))
 (segment (start 102.191356 78.405) (end 99.799558 78.405) (width 0.2) (layer "F.Cu") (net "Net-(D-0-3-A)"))
 (segment (start 106.812455 73.783901) (end 102.191356 78.405) (width 0.2) (layer "F.Cu") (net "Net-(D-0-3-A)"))
 (via (at 106.982603 70.949197) (size 0.6) (drill 0.3) (layers "F.Cu" "B.Cu") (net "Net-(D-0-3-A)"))
 (segment (start 86.445839 76.070254) (end 83.020254 76.070254) (width 0.2) (layer "F.Cu") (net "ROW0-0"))
 (segment (start 108.02147 64.458501) (end 108.985364 62.788987) (width 0.2) (layer "F.Cu") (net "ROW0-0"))
 (segment (start 98.836091 69.65) (end 98.030942 69.65) (width 0.2) (layer "F.Cu") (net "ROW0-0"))
 (segment (start 104.290974 59.469911) (end 102.685894 59.899994) (width 0.2) (layer "F.Cu") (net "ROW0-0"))
 (segment (start 98.030942 69.65) (end 96.104022 71.57692) (width 0.2) (layer "F.Cu") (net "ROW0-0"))
 (segment (start 106.792047 64.787929) (end 106.588068 64.991908) (width 0.2) (layer "F.Cu") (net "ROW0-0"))
 (segment (start 96.104022 71.57692) (end 90.939173 71.57692) (width 0.2) (layer "F.Cu") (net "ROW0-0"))
 (segment (start 90.939173 71.57692) (end 86.445839 76.070254) (width 0.2) (layer "F.Cu") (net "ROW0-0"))
 (segment (start 108.985364 62.788987) (end 108.792396 62.068808) (width 0.2) (layer "F.Cu") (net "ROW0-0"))
 (segment (start 103.494183 64.991908) (end 98.836091 69.65) (width 0.2) (layer "F.Cu") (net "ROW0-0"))
 (segment (start 83.020254 76.070254) (end 82.65 75.7) (width 0.2) (layer "F.Cu") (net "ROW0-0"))
 (segment (start 106.792039 64.787926) (end 108.02147 64.458501) (width 0.2) (layer "F.Cu") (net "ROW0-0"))
 (segment (start 106.588068 64.991908) (end 103.494183 64.991908) (width 0.2) (layer "F.Cu") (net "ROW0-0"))
 (segment (start 108.792396 62.068808) (end 104.290974 59.469911) (width 0.2) (layer "F.Cu") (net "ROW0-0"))
 (via (at 82.65 75.7) (size 0.6) (drill 0.3) (layers "F.Cu" "B.Cu") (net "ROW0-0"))
 (segment (start 46.046955 79.82548) (end 45.704498 80.167937) (width 0.2) (layer "B.Cu") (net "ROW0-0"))
 (segment (start 73.912476 72.46) (end 59.891746 72.46) (width 0.2) (layer "B.Cu") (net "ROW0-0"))
 (segment (start 81.4 74.45) (end 75.902476 74.45) (width 0.2) (layer "B.Cu") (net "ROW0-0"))
 (segment (start 75.902476 74.45) (end 73.912476 72.46) (width 0.2) (layer "B.Cu") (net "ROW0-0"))
 (segment (start 52.526266 79.82548) (end 46.046955 79.82548) (width 0.2) (layer "B.Cu") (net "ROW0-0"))
 (segment (start 59.891746 72.46) (end 52.526266 79.82548) (width 0.2) (layer "B.Cu") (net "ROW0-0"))
 (segment (start 82.65 75.7) (end 81.4 74.45) (width 0.2) (layer "B.Cu") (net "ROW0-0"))
 (segment (start 57.602608 71.83133) (end 56.558816 70.787538) (width 0.2) (layer "F.Cu") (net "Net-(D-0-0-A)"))
 (segment (start 57.602608 73.42856) (end 57.602608 71.83133) (width 0.2) (layer "F.Cu") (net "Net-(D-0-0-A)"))
 (segment (start 57.602608 76.524957) (end 53.295502 80.832063) (width 0.2) (layer "F.Cu") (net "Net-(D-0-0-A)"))
 (segment (start 57.602608 73.42856) (end 57.602608 76.524957) (width 0.2) (layer "F.Cu") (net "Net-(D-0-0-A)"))
 (via (at 56.558816 70.787538) (size 0.6) (drill 0.3) (layers "F.Cu" "B.Cu") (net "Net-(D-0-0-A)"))
 (segment (start 109.135879 61.805233) (end 103.496956 58.549606) (width 0.2) (layer "F.Cu") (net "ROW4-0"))
 (segment (start 101.957164 58.962188) (end 101.093262 60.458499) (width 0.2) (layer "F.Cu") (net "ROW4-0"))
 (segment (start 109.670839 63.801721) (end 109.135879 61.805233) (width 0.2) (layer "F.Cu") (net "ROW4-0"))
 (segment (start 103.496956 58.549606) (end 101.957164 58.962188) (width 0.2) (layer "F.Cu") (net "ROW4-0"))
 (segment (start 101.093262 60.458499) (end 99.863844 60.787923) (width 0.2) (layer "F.Cu") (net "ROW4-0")))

